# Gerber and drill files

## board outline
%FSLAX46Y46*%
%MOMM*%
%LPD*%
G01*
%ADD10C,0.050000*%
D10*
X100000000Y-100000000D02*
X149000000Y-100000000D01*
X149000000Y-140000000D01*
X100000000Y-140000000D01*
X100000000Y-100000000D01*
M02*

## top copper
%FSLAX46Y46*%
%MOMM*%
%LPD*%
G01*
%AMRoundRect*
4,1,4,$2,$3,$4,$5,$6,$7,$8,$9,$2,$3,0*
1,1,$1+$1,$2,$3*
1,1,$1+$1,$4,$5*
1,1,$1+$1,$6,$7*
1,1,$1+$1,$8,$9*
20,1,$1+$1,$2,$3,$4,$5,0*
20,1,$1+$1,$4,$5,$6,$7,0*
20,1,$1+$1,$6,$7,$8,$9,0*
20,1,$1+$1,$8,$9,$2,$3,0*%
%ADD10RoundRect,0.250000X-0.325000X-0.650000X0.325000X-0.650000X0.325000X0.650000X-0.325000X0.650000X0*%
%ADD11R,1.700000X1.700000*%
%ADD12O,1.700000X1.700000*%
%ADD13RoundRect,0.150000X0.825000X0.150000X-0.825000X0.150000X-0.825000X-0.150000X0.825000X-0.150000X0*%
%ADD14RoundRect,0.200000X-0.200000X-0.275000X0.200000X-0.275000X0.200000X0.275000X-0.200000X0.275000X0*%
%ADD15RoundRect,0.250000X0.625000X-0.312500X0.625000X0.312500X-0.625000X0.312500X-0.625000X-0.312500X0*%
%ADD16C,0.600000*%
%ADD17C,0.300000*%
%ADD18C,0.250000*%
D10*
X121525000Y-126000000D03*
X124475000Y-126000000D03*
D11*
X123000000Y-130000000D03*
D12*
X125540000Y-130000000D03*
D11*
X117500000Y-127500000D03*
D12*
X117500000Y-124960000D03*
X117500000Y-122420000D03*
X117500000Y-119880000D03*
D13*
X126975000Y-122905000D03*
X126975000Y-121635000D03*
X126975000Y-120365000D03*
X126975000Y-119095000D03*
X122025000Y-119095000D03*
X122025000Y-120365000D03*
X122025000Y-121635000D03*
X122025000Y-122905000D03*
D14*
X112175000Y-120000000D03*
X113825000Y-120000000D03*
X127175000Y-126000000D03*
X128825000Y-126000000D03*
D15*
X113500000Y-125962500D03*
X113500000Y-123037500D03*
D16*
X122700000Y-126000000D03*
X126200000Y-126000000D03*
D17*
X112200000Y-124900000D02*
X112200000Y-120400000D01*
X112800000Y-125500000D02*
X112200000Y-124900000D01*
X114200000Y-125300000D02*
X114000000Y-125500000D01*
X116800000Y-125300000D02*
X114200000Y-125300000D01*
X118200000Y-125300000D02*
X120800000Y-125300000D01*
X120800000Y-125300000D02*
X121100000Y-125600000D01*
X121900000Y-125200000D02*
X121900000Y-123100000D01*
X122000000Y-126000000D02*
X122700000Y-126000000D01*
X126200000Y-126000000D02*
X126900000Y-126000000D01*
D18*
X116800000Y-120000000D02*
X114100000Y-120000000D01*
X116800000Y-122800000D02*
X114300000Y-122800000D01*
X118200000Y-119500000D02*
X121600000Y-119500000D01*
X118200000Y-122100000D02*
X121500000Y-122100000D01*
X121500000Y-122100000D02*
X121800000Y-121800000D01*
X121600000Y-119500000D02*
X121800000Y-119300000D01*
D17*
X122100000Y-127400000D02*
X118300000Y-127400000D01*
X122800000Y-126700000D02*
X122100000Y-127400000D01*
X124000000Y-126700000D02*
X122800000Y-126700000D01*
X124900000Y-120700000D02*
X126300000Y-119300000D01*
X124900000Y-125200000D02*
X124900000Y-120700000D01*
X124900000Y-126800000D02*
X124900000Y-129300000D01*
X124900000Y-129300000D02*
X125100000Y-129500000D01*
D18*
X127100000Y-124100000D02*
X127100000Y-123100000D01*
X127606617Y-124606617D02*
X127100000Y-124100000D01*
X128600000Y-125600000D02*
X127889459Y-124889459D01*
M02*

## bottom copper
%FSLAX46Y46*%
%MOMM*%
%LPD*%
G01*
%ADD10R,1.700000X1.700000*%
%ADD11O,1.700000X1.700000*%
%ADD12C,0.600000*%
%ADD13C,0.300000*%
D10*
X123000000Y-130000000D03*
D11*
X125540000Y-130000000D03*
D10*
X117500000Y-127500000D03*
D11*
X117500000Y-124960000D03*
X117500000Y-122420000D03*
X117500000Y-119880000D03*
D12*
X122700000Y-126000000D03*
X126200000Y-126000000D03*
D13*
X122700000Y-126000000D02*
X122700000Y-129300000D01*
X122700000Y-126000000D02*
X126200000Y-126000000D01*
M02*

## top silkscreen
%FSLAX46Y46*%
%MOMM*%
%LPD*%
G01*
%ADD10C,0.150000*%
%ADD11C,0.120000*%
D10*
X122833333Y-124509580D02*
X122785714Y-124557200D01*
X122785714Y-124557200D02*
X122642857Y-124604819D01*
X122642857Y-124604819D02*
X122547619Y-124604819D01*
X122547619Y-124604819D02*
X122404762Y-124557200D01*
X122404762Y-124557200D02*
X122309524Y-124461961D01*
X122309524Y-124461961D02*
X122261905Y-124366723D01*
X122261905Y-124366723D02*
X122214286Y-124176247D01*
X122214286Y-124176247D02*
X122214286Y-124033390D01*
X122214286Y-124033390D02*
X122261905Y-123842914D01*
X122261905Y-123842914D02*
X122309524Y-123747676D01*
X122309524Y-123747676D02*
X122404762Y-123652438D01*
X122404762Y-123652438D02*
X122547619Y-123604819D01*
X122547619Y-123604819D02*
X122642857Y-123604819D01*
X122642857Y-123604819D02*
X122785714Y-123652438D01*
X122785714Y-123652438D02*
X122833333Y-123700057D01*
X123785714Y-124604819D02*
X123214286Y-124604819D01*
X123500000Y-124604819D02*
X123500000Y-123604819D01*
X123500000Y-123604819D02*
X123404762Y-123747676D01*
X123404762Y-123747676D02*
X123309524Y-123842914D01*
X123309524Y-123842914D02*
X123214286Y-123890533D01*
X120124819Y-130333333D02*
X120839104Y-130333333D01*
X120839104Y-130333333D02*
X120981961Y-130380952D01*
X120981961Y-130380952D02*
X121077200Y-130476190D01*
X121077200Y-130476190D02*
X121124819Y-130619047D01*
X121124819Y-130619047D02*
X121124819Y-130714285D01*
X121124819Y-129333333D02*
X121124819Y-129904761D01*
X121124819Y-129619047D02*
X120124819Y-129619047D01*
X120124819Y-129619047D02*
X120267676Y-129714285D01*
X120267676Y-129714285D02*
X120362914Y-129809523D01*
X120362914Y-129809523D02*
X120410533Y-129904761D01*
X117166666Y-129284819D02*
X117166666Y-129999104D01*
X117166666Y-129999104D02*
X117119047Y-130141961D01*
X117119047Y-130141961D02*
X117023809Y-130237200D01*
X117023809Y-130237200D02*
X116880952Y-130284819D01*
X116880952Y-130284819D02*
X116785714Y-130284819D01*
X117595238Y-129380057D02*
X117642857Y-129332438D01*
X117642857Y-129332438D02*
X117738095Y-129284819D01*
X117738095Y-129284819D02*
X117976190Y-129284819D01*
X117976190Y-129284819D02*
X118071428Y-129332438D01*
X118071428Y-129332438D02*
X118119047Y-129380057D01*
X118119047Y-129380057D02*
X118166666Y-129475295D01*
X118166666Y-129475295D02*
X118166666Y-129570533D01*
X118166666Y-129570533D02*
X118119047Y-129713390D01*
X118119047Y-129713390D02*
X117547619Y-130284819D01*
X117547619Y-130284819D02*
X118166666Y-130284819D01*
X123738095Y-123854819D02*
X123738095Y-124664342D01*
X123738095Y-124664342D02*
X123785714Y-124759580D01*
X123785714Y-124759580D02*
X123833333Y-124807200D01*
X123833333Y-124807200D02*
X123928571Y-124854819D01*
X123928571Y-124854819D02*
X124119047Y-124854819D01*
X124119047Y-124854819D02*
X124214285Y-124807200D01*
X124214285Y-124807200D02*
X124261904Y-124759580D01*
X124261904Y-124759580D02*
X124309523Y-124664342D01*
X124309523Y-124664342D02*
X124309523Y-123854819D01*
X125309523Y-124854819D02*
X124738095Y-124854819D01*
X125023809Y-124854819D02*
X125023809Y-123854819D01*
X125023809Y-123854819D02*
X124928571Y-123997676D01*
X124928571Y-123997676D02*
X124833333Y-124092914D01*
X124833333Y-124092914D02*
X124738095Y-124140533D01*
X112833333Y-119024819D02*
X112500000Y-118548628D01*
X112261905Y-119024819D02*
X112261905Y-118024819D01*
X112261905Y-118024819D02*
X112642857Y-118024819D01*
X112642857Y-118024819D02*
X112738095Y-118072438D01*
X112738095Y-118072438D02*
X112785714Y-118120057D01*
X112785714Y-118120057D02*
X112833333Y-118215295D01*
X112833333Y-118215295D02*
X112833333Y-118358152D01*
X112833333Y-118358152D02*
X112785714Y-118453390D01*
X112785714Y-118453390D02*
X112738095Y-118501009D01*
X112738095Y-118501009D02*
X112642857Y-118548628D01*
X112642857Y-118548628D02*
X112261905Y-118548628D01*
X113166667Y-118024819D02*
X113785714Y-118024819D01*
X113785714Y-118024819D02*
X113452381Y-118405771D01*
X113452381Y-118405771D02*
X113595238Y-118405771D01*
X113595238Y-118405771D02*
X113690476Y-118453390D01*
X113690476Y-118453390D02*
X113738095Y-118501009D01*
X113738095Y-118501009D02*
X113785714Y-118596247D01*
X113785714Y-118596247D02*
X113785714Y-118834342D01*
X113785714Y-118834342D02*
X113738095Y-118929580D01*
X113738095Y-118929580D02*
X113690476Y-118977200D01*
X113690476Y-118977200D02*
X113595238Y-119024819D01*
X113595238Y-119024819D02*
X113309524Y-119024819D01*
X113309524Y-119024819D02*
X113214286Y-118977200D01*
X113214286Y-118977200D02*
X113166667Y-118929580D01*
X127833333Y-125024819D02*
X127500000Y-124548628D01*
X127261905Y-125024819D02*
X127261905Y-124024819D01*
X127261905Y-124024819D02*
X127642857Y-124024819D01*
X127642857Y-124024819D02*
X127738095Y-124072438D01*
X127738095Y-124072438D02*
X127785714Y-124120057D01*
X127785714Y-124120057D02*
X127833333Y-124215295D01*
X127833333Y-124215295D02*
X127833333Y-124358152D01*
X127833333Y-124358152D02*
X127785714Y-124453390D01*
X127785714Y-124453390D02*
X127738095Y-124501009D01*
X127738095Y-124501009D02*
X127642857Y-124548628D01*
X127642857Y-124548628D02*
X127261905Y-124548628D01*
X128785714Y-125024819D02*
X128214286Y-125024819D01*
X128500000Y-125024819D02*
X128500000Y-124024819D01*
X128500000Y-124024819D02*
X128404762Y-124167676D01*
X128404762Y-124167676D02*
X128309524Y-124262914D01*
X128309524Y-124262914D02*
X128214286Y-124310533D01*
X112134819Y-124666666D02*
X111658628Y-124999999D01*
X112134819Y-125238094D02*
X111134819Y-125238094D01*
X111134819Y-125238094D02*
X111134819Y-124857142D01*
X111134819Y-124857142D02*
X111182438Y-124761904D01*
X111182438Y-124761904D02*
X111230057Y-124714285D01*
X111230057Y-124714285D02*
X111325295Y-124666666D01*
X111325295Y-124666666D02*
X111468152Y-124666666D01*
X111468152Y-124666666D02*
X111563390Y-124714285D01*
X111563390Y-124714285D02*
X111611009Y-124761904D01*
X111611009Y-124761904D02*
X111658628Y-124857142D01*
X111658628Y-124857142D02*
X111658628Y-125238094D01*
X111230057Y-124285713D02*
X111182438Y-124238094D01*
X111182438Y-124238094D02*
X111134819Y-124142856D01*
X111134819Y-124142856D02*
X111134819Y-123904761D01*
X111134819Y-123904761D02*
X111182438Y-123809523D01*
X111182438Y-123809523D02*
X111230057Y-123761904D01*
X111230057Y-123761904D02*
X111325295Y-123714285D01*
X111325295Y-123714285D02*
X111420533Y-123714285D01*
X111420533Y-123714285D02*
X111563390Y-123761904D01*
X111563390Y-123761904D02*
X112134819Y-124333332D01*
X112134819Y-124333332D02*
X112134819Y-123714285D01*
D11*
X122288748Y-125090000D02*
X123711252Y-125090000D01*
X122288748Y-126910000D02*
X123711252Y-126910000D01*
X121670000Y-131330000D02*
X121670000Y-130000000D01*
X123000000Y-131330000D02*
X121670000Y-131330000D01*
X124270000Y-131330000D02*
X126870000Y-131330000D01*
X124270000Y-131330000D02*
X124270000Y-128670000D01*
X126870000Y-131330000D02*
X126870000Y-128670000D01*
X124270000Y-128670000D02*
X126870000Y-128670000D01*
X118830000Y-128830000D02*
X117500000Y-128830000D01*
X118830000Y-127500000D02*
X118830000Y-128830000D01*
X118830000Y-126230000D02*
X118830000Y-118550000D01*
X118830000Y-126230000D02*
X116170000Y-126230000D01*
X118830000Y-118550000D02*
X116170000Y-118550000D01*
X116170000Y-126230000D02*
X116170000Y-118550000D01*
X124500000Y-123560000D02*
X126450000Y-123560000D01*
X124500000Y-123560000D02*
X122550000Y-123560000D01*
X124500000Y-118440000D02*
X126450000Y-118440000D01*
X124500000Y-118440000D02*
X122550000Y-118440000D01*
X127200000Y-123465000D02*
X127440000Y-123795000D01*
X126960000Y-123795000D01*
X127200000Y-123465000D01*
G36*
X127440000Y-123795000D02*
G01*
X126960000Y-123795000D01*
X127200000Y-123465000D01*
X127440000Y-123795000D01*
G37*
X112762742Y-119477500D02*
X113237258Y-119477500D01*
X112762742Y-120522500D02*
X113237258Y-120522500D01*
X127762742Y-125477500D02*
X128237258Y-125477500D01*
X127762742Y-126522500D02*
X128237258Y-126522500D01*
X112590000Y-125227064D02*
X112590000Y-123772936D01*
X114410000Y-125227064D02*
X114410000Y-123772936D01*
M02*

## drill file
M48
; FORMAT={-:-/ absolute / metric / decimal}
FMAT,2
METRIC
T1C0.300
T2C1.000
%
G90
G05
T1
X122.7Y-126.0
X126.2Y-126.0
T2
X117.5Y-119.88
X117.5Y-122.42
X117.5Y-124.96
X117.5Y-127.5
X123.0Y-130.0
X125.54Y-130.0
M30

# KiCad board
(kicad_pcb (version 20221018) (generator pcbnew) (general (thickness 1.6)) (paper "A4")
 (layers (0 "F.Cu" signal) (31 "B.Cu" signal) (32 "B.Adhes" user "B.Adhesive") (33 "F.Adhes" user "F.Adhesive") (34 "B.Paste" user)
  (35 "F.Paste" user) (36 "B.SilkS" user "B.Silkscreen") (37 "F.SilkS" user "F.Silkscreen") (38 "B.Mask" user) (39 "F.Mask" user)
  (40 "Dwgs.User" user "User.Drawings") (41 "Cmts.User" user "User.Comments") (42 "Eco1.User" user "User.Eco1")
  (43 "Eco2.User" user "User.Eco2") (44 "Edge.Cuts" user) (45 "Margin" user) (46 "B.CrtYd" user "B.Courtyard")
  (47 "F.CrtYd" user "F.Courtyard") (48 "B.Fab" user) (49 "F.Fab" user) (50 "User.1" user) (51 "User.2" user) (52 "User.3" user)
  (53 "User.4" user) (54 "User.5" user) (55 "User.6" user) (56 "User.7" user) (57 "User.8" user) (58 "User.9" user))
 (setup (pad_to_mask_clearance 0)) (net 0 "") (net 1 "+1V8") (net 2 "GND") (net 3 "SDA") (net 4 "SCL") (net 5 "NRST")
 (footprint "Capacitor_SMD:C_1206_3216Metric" (layer "F.Cu") (at 123 126)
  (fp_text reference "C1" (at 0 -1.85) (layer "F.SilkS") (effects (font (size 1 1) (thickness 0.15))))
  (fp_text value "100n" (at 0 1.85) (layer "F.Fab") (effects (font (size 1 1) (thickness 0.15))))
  (fp_line (start -0.711252 -0.91) (end 0.711252 -0.91) (stroke (width 0.12) (type solid)) (layer "F.SilkS"))
  (fp_line (start -0.711252 0.91) (end 0.711252 0.91) (stroke (width 0.12) (type solid)) (layer "F.SilkS"))
  (pad "1" smd roundrect (at -1.475 0) (size 1.15 1.8) (layers "F.Cu" "F.Paste" "F.Mask") (roundrect_rratio 0.217391) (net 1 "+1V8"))
  (pad "2" smd roundrect (at 1.475 0) (size 1.15 1.8) (layers "F.Cu" "F.Paste" "F.Mask") (roundrect_rratio 0.217391) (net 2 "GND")))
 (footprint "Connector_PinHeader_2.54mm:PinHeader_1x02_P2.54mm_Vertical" (layer "F.Cu") (at 123 130 90)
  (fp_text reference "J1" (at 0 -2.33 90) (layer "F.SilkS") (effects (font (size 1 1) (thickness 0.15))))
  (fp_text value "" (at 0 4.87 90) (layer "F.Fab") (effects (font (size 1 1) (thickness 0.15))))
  (fp_line (start -1.33 -1.33) (end 0 -1.33) (stroke (width 0.12) (type solid)) (layer "F.SilkS"))
  (fp_line (start -1.33 0) (end -1.33 -1.33) (stroke (width 0.12) (type solid)) (layer "F.SilkS"))
  (fp_line (start -1.33 1.27) (end -1.33 3.87) (stroke (width 0.12) (type solid)) (layer "F.SilkS"))
  (fp_line (start -1.33 1.27) (end 1.33 1.27) (stroke (width 0.12) (type solid)) (layer "F.SilkS"))
  (fp_line (start -1.33 3.87) (end 1.33 3.87) (stroke (width 0.12) (type solid)) (layer "F.SilkS"))
  (fp_line (start 1.33 1.27) (end 1.33 3.87) (stroke (width 0.12) (type solid)) (layer "F.SilkS"))
  (pad "1" thru_hole rect (at 0 0 90) (size 1.7 1.7) (drill 1) (layers "*.Cu" "*.Mask") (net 1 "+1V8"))
  (pad "2" thru_hole oval (at 0 2.54 90) (size 1.7 1.7) (drill 1) (layers "*.Cu" "*.Mask") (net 2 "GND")))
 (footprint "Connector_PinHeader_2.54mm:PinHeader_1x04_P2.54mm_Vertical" (layer "F.Cu") (at 117.5 127.5 180)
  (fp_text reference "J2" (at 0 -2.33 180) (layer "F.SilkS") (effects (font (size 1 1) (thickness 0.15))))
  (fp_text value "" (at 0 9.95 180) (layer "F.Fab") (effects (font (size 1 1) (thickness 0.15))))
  (fp_line (start -1.33 -1.33) (end 0 -1.33) (stroke (width 0.12) (type solid)) (layer "F.SilkS"))
  (fp_line (start -1.33 0) (end -1.33 -1.33) (stroke (width 0.12) (type solid)) (layer "F.SilkS"))
  (fp_line (start -1.33 1.27) (end -1.33 8.95) (stroke (width 0.12) (type solid)) (layer "F.SilkS"))
  (fp_line (start -1.33 1.27) (end 1.33 1.27) (stroke (width 0.12) (type solid)) (layer "F.SilkS"))
  (fp_line (start -1.33 8.95) (end 1.33 8.95) (stroke (width 0.12) (type solid)) (layer "F.SilkS"))
  (fp_line (start 1.33 1.27) (end 1.33 8.95) (stroke (width 0.12) (type solid)) (layer "F.SilkS"))
  (pad "1" thru_hole rect (at 0 0 180) (size 1.7 1.7) (drill 1) (layers "*.Cu" "*.Mask") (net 2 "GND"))
  (pad "2" thru_hole oval (at 0 2.54 180) (size 1.7 1.7) (drill 1) (layers "*.Cu" "*.Mask") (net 1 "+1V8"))
  (pad "3" thru_hole oval (at 0 5.08 180) (size 1.7 1.7) (drill 1) (layers "*.Cu" "*.Mask") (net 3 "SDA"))
  (pad "4" thru_hole oval (at 0 7.62 180) (size 1.7 1.7) (drill 1) (layers "*.Cu" "*.Mask") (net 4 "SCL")))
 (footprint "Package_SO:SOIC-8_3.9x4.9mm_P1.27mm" (layer "F.Cu") (at 124.5 121 180)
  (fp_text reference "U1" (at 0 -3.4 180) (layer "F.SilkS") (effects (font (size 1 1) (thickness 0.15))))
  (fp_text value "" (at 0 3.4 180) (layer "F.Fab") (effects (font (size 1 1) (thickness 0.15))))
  (fp_line (start 0 -2.56) (end -1.95 -2.56) (stroke (width 0.12) (type solid)) (layer "F.SilkS"))
  (fp_line (start 0 -2.56) (end 1.95 -2.56) (stroke (width 0.12) (type solid)) (layer "F.SilkS"))
  (fp_line (start 0 2.56) (end -1.95 2.56) (stroke (width 0.12) (type solid)) (layer "F.SilkS"))
  (fp_line (start 0 2.56) (end 1.95 2.56) (stroke (width 0.12) (type solid)) (layer "F.SilkS"))
  (fp_poly
   (pts (xy -2.7 -2.465) (xy -2.94 -2.795) (xy -2.46 -2.795) (xy -2.7 -2.465)) (stroke (width 0.12) (type solid)) (fill solid)
   (layer "F.SilkS"))
  (pad "1" smd roundrect (at -2.475 -1.905 180) (size 1.95 0.6) (layers "F.Cu" "F.Paste" "F.Mask") (roundrect_rratio 0.25) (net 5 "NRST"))
  (pad "2" smd roundrect (at -2.475 -0.635 180) (size 1.95 0.6) (layers "F.Cu" "F.Paste" "F.Mask") (roundrect_rratio 0.25))
  (pad "3" smd roundrect (at -2.475 0.635 180) (size 1.95 0.6) (layers "F.Cu" "F.Paste" "F.Mask") (roundrect_rratio 0.25))
  (pad "4" smd roundrect (at -2.475 1.905 180) (size 1.95 0.6) (layers "F.Cu" "F.Paste" "F.Mask") (roundrect_rratio 0.25) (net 2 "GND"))
  (pad "5" smd roundrect (at 2.475 1.905 180) (size 1.95 0.6) (layers "F.Cu" "F.Paste" "F.Mask") (roundrect_rratio 0.25) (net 4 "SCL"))
  (pad "6" smd roundrect (at 2.475 0.635 180) (size 1.95 0.6) (layers "F.Cu" "F.Paste" "F.Mask") (roundrect_rratio 0.25))
  (pad "7" smd roundrect (at 2.475 -0.635 180) (size 1.95 0.6) (layers "F.Cu" "F.Paste" "F.Mask") (roundrect_rratio 0.25) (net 3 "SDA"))
  (pad "8" smd roundrect (at 2.475 -1.905 180) (size 1.95 0.6) (layers "F.Cu" "F.Paste" "F.Mask") (roundrect_rratio 0.25) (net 1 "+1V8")))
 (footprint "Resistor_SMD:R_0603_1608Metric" (layer "F.Cu") (at 113 120)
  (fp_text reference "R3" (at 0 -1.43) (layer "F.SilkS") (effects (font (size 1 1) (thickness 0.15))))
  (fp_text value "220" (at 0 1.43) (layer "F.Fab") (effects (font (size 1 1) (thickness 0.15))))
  (fp_line (start -0.237258 -0.5225) (end 0.237258 -0.5225) (stroke (width 0.12) (type solid)) (layer "F.SilkS"))
  (fp_line (start -0.237258 0.5225) (end 0.237258 0.5225) (stroke (width 0.12) (type solid)) (layer "F.SilkS"))
  (pad "1" smd roundrect (at -0.825 0) (size 0.8 0.95) (layers "F.Cu" "F.Paste" "F.Mask") (roundrect_rratio 0.25) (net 1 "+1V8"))
  (pad "2" smd roundrect (at 0.825 0) (size 0.8 0.95) (layers "F.Cu" "F.Paste" "F.Mask") (roundrect_rratio 0.25) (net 4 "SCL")))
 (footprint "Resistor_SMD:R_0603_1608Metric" (layer "F.Cu") (at 128 126)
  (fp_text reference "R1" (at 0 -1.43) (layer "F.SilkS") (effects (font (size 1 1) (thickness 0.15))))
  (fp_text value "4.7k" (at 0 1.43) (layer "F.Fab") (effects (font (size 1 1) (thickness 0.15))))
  (fp_line (start -0.237258 -0.5225) (end 0.237258 -0.5225) (stroke (width 0.12) (type solid)) (layer "F.SilkS"))
  (fp_line (start -0.237258 0.5225) (end 0.237258 0.5225) (stroke (width 0.12) (type solid)) (layer "F.SilkS"))
  (pad "1" smd roundrect (at -0.825 0) (size 0.8 0.95) (layers "F.Cu" "F.Paste" "F.Mask") (roundrect_rratio 0.25) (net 1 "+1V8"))
  (pad "2" smd roundrect (at 0.825 0) (size 0.8 0.95) (layers "F.Cu" "F.Paste" "F.Mask") (roundrect_rratio 0.25) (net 5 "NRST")))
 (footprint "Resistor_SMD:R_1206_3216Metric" (layer "F.Cu") (at 113.5 124.5 90)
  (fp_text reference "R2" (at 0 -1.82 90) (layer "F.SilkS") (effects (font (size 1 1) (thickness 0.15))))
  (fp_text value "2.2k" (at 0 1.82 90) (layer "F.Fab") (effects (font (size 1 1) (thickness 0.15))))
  (fp_line (start -0.727064 -0.91) (end 0.727064 -0.91) (stroke (width 0.12) (type solid)) (layer "F.SilkS"))
  (fp_line (start -0.727064 0.91) (end 0.727064 0.91) (stroke (width 0.12) (type solid)) (layer "F.SilkS"))
  (pad "1" smd roundrect (at -1.4625 0 90) (size 1.125 1.75) (layers "F.Cu" "F.Paste" "F.Mask") (roundrect_rratio 0.222222) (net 1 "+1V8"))
  (pad "2" smd roundrect (at 1.4625 0 90) (size 1.125 1.75) (layers "F.Cu" "F.Paste" "F.Mask") (roundrect_rratio 0.222222) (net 3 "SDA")))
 (gr_rect (start 100 100) (end 149 140) (stroke (width 0.05) (type default)) (fill none) (layer "Edge.Cuts"))
 (segment (start 112.2 124.9) (end 112.2 120.4) (width 0.3) (layer "F.Cu") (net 1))
 (segment (start 112.8 125.5) (end 112.2 124.9) (width 0.3) (layer "F.Cu") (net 1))
 (segment (start 114.2 125.3) (end 114 125.5) (width 0.3) (layer "F.Cu") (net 1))
 (segment (start 116.8 125.3) (end 114.2 125.3) (width 0.3) (layer "F.Cu") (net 1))
 (segment (start 118.2 125.3) (end 120.8 125.3) (width 0.3) (layer "F.Cu") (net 1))
 (segment (start 120.8 125.3) (end 121.1 125.6) (width 0.3) (layer "F.Cu") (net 1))
 (segment (start 121.9 125.2) (end 121.9 123.1) (width 0.3) (layer "F.Cu") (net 1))
 (segment (start 122 126) (end 122.7 126) (width 0.3) (layer "F.Cu") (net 1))
 (segment (start 126.2 126) (end 126.9 126) (width 0.3) (layer "F.Cu") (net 1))
 (via (at 122.7 126) (size 0.6) (drill 0.3) (layers "F.Cu" "B.Cu") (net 1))
 (via (at 126.2 126) (size 0.6) (drill 0.3) (layers "F.Cu" "B.Cu") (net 1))
 (segment (start 116.8 120) (end 114.1 120) (width 0.25) (layer "F.Cu") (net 4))
 (segment (start 116.8 122.8) (end 114.3 122.8) (width 0.25) (layer "F.Cu") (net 3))
 (segment (start 118.2 119.5) (end 121.6 119.5) (width 0.25) (layer "F.Cu") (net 4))
 (segment (start 118.2 122.1) (end 121.5 122.1) (width 0.25) (layer "F.Cu") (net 3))
 (segment (start 121.5 122.1) (end 121.8 121.8) (width 0.25) (layer "F.Cu") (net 3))
 (segment (start 121.6 119.5) (end 121.8 119.3) (width 0.25) (layer "F.Cu") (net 4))
 (segment (start 122.1 127.4) (end 118.3 127.4) (width 0.3) (layer "F.Cu") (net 2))
 (segment (start 122.7 126) (end 122.7 129.3) (width 0.3) (layer "B.Cu") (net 1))
 (segment (start 122.7 126) (end 126.2 126) (width 0.3) (layer "B.Cu") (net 1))
 (segment (start 122.8 126.7) (end 122.1 127.4) (width 0.3) (layer "F.Cu") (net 2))
 (segment (start 124 126.7) (end 122.8 126.7) (width 0.3) (layer "F.Cu") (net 2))
 (segment (start 124.9 120.7) (end 126.3 119.3) (width 0.3) (layer "F.Cu") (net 2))
 (segment (start 124.9 125.2) (end 124.9 120.7) (width 0.3) (layer "F.Cu") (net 2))
 (segment (start 124.9 126.8) (end 124.9 129.3) (width 0.3) (layer "F.Cu") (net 2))
 (segment (start 124.9 129.3) (end 125.1 129.5) (width 0.3) (layer "F.Cu") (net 2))
 (segment (start 127.1 124.1) (end 127.1 123.1) (width 0.25) (layer "F.Cu") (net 5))
 (segment (start 127.606617 124.606617) (end 127.1 124.1) (width 0.25) (layer "F.Cu") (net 5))
 (segment (start 128.6 125.6) (end 127.889459 124.889459) (width 0.25) (layer "F.Cu") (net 5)))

